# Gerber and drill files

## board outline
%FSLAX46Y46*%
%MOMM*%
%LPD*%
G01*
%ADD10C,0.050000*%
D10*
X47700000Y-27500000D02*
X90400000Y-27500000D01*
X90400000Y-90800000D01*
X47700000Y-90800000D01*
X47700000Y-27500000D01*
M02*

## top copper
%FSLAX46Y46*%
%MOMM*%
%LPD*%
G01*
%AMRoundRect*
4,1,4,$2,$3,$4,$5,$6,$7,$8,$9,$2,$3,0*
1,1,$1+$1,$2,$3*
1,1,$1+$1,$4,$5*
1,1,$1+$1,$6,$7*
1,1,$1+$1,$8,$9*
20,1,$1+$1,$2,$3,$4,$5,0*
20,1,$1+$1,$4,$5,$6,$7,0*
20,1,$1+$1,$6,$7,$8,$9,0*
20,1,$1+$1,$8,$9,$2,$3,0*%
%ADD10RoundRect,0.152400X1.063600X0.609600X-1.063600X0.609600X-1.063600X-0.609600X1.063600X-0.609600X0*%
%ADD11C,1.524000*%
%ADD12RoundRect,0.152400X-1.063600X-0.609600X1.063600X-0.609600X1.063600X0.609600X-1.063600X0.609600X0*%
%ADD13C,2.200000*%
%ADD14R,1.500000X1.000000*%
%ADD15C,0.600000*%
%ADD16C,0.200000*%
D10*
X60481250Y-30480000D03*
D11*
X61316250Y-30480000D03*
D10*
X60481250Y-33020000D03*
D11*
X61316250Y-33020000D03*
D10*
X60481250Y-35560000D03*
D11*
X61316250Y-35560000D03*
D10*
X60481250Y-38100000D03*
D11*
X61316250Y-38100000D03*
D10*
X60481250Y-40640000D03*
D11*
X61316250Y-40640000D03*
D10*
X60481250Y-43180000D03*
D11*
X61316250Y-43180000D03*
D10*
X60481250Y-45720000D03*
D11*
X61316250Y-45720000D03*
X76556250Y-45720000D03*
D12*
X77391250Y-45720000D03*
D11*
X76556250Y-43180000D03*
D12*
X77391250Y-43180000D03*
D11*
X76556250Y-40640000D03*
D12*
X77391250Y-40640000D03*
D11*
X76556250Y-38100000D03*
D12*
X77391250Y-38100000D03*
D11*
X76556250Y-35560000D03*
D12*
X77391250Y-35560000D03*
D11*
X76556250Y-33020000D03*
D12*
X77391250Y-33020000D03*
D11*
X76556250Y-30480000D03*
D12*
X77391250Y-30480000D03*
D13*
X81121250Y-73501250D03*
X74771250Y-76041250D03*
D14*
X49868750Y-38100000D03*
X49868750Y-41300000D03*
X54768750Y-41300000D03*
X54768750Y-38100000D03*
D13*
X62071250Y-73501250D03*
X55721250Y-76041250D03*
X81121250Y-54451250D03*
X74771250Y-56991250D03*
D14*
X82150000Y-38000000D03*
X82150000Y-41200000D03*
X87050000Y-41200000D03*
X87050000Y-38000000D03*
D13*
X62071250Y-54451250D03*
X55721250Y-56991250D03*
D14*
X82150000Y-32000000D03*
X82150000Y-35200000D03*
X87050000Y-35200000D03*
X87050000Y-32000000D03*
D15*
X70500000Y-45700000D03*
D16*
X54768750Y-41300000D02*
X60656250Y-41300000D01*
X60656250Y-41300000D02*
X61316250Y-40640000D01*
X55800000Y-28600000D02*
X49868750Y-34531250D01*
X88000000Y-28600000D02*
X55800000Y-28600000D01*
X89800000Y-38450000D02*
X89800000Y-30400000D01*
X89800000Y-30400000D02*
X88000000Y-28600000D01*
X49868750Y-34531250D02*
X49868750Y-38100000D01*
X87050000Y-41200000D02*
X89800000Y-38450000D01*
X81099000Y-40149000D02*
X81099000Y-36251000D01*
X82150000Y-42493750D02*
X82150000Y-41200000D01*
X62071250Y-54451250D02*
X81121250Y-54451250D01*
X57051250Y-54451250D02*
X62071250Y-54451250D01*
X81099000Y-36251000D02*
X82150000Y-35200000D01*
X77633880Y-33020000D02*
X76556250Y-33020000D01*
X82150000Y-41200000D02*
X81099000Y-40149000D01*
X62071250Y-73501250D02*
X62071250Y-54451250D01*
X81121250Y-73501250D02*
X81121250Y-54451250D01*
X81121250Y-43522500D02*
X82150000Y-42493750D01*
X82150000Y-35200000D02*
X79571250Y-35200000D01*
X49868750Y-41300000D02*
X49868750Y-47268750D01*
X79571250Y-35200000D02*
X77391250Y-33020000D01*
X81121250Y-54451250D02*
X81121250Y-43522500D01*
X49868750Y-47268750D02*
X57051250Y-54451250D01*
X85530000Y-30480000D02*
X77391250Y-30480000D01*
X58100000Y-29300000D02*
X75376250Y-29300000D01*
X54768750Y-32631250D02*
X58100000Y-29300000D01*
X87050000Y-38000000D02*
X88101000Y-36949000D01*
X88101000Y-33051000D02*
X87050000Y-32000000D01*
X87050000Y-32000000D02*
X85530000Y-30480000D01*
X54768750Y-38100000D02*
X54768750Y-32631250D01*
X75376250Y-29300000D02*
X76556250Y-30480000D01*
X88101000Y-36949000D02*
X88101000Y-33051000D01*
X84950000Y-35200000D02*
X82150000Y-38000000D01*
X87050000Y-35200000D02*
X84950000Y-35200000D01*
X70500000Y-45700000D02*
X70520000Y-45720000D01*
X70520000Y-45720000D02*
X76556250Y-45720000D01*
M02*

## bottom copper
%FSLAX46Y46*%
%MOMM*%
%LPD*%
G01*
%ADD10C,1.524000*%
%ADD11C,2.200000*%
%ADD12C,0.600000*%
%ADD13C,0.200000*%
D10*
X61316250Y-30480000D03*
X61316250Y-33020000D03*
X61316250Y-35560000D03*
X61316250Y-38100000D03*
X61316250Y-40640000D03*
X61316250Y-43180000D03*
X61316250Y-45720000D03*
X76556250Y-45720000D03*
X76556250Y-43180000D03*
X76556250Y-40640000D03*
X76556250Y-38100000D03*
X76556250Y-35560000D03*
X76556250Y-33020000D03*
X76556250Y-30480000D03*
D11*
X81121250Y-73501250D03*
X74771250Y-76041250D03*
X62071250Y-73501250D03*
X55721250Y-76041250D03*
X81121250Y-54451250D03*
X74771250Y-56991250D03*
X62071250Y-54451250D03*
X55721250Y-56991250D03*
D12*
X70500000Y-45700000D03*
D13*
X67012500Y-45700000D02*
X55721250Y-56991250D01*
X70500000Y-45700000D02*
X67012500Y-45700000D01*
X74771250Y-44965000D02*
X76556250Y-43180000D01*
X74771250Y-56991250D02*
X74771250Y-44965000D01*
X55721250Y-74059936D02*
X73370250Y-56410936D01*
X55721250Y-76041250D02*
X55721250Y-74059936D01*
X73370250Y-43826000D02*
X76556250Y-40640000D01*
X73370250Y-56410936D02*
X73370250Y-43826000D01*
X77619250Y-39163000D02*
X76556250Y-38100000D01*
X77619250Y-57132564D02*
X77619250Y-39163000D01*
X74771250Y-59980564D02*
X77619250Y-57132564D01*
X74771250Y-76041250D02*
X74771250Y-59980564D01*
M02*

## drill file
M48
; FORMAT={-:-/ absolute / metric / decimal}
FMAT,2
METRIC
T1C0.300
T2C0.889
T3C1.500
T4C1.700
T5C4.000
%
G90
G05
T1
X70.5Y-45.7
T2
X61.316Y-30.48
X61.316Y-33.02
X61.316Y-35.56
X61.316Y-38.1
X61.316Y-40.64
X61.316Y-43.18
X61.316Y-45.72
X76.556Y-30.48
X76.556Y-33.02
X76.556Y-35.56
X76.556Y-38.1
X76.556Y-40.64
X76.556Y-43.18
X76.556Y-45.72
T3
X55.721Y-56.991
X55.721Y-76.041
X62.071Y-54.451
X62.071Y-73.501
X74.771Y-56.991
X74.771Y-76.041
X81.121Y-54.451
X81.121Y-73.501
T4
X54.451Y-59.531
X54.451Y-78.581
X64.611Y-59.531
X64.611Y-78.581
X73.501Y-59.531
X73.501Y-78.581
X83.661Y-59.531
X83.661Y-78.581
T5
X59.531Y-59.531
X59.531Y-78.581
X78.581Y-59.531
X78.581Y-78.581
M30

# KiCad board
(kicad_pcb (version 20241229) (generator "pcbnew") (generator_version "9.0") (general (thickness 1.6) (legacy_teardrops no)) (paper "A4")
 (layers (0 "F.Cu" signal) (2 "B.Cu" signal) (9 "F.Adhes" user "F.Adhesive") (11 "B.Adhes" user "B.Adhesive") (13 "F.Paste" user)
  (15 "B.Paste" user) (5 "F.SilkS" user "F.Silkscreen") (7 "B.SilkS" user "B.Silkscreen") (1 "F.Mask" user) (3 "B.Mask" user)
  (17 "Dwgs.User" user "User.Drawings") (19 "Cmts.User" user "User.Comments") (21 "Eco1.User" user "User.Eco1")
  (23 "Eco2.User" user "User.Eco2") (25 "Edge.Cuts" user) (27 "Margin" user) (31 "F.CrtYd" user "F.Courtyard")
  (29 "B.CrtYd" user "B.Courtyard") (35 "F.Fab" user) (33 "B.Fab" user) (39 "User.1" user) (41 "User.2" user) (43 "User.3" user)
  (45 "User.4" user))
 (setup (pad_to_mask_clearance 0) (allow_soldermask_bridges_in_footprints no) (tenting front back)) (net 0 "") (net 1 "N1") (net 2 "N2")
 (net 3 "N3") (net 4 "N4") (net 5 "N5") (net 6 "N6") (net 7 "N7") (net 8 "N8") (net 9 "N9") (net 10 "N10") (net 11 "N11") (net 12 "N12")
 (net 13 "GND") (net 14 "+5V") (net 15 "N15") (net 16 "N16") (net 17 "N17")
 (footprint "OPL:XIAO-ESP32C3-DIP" (layer "F.Cu") (at 69.05625 38.1)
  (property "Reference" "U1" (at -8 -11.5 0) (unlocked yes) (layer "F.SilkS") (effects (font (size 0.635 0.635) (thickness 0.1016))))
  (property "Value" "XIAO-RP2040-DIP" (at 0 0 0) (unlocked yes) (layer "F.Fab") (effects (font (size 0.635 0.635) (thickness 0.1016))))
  (pad "1" smd roundrect (at -8.575 -7.62 180) (size 2.432 1.524) (layers "F.Cu" "F.Mask") (roundrect_rratio 0.1) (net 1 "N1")
   (thermal_bridge_angle 45))
  (pad "1" thru_hole circle (at -7.74 -7.62 180) (size 1.524 1.524) (drill 0.889) (layers "*.Cu" "*.Mask") (remove_unused_layers no)
   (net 1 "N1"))
  (pad "2" smd roundrect (at -8.575 -5.08 180) (size 2.432 1.524) (layers "F.Cu" "F.Mask") (roundrect_rratio 0.1) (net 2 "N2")
   (thermal_bridge_angle 45))
  (pad "2" thru_hole circle (at -7.74 -5.08 180) (size 1.524 1.524) (drill 0.889) (layers "*.Cu" "*.Mask") (remove_unused_layers no)
   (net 2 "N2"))
  (pad "3" smd roundrect (at -8.575 -2.54 180) (size 2.432 1.524) (layers "F.Cu" "F.Mask") (roundrect_rratio 0.1) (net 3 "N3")
   (thermal_bridge_angle 45))
  (pad "3" thru_hole circle (at -7.74 -2.54 180) (size 1.524 1.524) (drill 0.889) (layers "*.Cu" "*.Mask") (remove_unused_layers no)
   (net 3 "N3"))
  (pad "4" smd roundrect (at -8.575 0 180) (size 2.432 1.524) (layers "F.Cu" "F.Mask") (roundrect_rratio 0.1) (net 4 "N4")
   (thermal_bridge_angle 45))
  (pad "4" thru_hole circle (at -7.74 0 180) (size 1.524 1.524) (drill 0.889) (layers "*.Cu" "*.Mask") (remove_unused_layers no)
   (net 4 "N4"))
  (pad "5" smd roundrect (at -8.575 2.54 180) (size 2.432 1.524) (layers "F.Cu" "F.Mask") (roundrect_rratio 0.1) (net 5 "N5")
   (thermal_bridge_angle 45))
  (pad "5" thru_hole circle (at -7.74 2.54 180) (size 1.524 1.524) (drill 0.889) (layers "*.Cu" "*.Mask") (remove_unused_layers no)
   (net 5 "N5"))
  (pad "6" smd roundrect (at -8.575 5.08 180) (size 2.432 1.524) (layers "F.Cu" "F.Mask") (roundrect_rratio 0.1) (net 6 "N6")
   (thermal_bridge_angle 45))
  (pad "6" thru_hole circle (at -7.74 5.08 180) (size 1.524 1.524) (drill 0.889) (layers "*.Cu" "*.Mask") (remove_unused_layers no)
   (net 6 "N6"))
  (pad "7" smd roundrect (at -8.575 7.62 180) (size 2.432 1.524) (layers "F.Cu" "F.Mask") (roundrect_rratio 0.1) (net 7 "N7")
   (thermal_bridge_angle 45))
  (pad "7" thru_hole circle (at -7.74 7.62 180) (size 1.524 1.524) (drill 0.889) (layers "*.Cu" "*.Mask") (remove_unused_layers no)
   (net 7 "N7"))
  (pad "8" thru_hole circle (at 7.5 7.62) (size 1.524 1.524) (drill 0.889) (layers "*.Cu" "*.Mask") (remove_unused_layers no) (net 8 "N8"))
  (pad "8" smd roundrect (at 8.335 7.62) (size 2.432 1.524) (layers "F.Cu" "F.Mask") (roundrect_rratio 0.1) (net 8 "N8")
   (thermal_bridge_angle 45))
  (pad "9" thru_hole circle (at 7.5 5.08) (size 1.524 1.524) (drill 0.889) (layers "*.Cu" "*.Mask") (remove_unused_layers no) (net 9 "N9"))
  (pad "9" smd roundrect (at 8.335 5.08) (size 2.432 1.524) (layers "F.Cu" "F.Mask") (roundrect_rratio 0.1) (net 9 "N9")
   (thermal_bridge_angle 45))
  (pad "10" thru_hole circle (at 7.5 2.54) (size 1.524 1.524) (drill 0.889) (layers "*.Cu" "*.Mask") (remove_unused_layers no)
   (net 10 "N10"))
  (pad "10" smd roundrect (at 8.335 2.54) (size 2.432 1.524) (layers "F.Cu" "F.Mask") (roundrect_rratio 0.1) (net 10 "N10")
   (thermal_bridge_angle 45))
  (pad "11" thru_hole circle (at 7.5 0) (size 1.524 1.524) (drill 0.889) (layers "*.Cu" "*.Mask") (remove_unused_layers no) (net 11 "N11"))
  (pad "11" smd roundrect (at 8.335 0) (size 2.432 1.524) (layers "F.Cu" "F.Mask") (roundrect_rratio 0.1) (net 11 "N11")
   (thermal_bridge_angle 45))
  (pad "12" thru_hole circle (at 7.5 -2.54) (size 1.524 1.524) (drill 0.889) (layers "*.Cu" "*.Mask") (remove_unused_layers no)
   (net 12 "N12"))
  (pad "12" smd roundrect (at 8.335 -2.54) (size 2.432 1.524) (layers "F.Cu" "F.Mask") (roundrect_rratio 0.1) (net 12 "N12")
   (thermal_bridge_angle 45))
  (pad "13" thru_hole circle (at 7.5 -5.08) (size 1.524 1.524) (drill 0.889) (layers "*.Cu" "*.Mask") (remove_unused_layers no)
   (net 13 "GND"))
  (pad "13" smd roundrect (at 8.335 -5.08) (size 2.432 1.524) (layers "F.Cu" "F.Mask") (roundrect_rratio 0.1) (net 13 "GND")
   (thermal_bridge_angle 45))
  (pad "14" thru_hole circle (at 7.5 -7.62) (size 1.524 1.524) (drill 0.889) (layers "*.Cu" "*.Mask") (remove_unused_layers no)
   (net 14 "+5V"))
  (pad "14" smd roundrect (at 8.335 -7.62) (size 2.432 1.524) (layers "F.Cu" "F.Mask") (roundrect_rratio 0.1) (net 14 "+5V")
   (thermal_bridge_angle 45)))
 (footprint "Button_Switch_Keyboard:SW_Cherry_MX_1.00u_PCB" (layer "F.Cu") (at 81.12125 73.50125)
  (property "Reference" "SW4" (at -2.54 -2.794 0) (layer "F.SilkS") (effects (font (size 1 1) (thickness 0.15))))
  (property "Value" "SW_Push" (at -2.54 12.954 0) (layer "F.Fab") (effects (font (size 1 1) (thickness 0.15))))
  (pad "" np_thru_hole circle (at -7.62 5.08) (size 1.7 1.7) (drill 1.7) (layers "*.Cu" "*.Mask"))
  (pad "" np_thru_hole circle (at -2.54 5.08) (size 4 4) (drill 4) (layers "*.Cu" "*.Mask"))
  (pad "" np_thru_hole circle (at 2.54 5.08) (size 1.7 1.7) (drill 1.7) (layers "*.Cu" "*.Mask"))
  (pad "1" thru_hole circle (at 0 0) (size 2.2 2.2) (drill 1.5) (layers "*.Cu" "*.Mask") (remove_unused_layers no) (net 13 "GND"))
  (pad "2" thru_hole circle (at -6.35 2.54) (size 2.2 2.2) (drill 1.5) (layers "*.Cu" "*.Mask") (remove_unused_layers no) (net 11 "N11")))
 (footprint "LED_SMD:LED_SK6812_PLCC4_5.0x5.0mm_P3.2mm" (layer "F.Cu") (at 52.31875 39.7)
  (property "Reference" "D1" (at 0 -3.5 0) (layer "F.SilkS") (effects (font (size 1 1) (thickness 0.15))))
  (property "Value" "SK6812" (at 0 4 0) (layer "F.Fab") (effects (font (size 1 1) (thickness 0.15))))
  (pad "1" smd rect (at -2.45 -1.6 180) (size 1.5 1) (layers "F.Cu" "F.Mask" "F.Paste") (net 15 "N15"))
  (pad "2" smd rect (at -2.45 1.6 180) (size 1.5 1) (layers "F.Cu" "F.Mask" "F.Paste") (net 13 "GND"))
  (pad "3" smd rect (at 2.45 1.6 180) (size 1.5 1) (layers "F.Cu" "F.Mask" "F.Paste") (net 5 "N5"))
  (pad "4" smd rect (at 2.45 -1.6 180) (size 1.5 1) (layers "F.Cu" "F.Mask" "F.Paste") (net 14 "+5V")))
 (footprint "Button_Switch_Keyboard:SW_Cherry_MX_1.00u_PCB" (layer "F.Cu") (at 62.07125 73.50125)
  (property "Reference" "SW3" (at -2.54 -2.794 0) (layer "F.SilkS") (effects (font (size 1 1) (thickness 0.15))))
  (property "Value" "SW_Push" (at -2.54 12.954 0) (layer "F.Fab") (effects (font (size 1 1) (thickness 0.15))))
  (pad "" np_thru_hole circle (at -7.62 5.08) (size 1.7 1.7) (drill 1.7) (layers "*.Cu" "*.Mask"))
  (pad "" np_thru_hole circle (at -2.54 5.08) (size 4 4) (drill 4) (layers "*.Cu" "*.Mask"))
  (pad "" np_thru_hole circle (at 2.54 5.08) (size 1.7 1.7) (drill 1.7) (layers "*.Cu" "*.Mask"))
  (pad "1" thru_hole circle (at 0 0) (size 2.2 2.2) (drill 1.5) (layers "*.Cu" "*.Mask") (remove_unused_layers no) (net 13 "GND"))
  (pad "2" thru_hole circle (at -6.35 2.54) (size 2.2 2.2) (drill 1.5) (layers "*.Cu" "*.Mask") (remove_unused_layers no) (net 10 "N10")))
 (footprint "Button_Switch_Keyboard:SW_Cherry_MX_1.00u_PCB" (layer "F.Cu") (at 81.12125 54.45125)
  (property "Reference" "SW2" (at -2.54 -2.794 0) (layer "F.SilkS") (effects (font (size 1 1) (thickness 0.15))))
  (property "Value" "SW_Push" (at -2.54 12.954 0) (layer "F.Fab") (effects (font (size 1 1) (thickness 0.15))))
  (pad "" np_thru_hole circle (at -7.62 5.08) (size 1.7 1.7) (drill 1.7) (layers "*.Cu" "*.Mask"))
  (pad "" np_thru_hole circle (at -2.54 5.08) (size 4 4) (drill 4) (layers "*.Cu" "*.Mask"))
  (pad "" np_thru_hole circle (at 2.54 5.08) (size 1.7 1.7) (drill 1.7) (layers "*.Cu" "*.Mask"))
  (pad "1" thru_hole circle (at 0 0) (size 2.2 2.2) (drill 1.5) (layers "*.Cu" "*.Mask") (remove_unused_layers no) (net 13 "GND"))
  (pad "2" thru_hole circle (at -6.35 2.54) (size 2.2 2.2) (drill 1.5) (layers "*.Cu" "*.Mask") (remove_unused_layers no) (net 9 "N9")))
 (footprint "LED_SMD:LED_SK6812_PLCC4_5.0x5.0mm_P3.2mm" (layer "F.Cu") (at 84.6 39.6)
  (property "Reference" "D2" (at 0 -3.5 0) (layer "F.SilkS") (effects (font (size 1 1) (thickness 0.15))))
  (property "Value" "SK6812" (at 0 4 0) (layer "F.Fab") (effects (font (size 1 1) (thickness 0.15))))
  (pad "1" smd rect (at -2.45 -1.6 180) (size 1.5 1) (layers "F.Cu" "F.Mask" "F.Paste") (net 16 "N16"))
  (pad "2" smd rect (at -2.45 1.6 180) (size 1.5 1) (layers "F.Cu" "F.Mask" "F.Paste") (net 13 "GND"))
  (pad "3" smd rect (at 2.45 1.6 180) (size 1.5 1) (layers "F.Cu" "F.Mask" "F.Paste") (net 15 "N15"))
  (pad "4" smd rect (at 2.45 -1.6 180) (size 1.5 1) (layers "F.Cu" "F.Mask" "F.Paste") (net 14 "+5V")))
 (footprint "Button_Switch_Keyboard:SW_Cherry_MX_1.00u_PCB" (layer "F.Cu") (at 62.07125 54.45125)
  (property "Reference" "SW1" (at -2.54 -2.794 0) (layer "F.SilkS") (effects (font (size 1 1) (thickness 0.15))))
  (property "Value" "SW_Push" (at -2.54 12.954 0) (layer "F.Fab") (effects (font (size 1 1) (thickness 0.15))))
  (pad "" np_thru_hole circle (at -7.62 5.08) (size 1.7 1.7) (drill 1.7) (layers "*.Cu" "*.Mask"))
  (pad "" np_thru_hole circle (at -2.54 5.08) (size 4 4) (drill 4) (layers "*.Cu" "*.Mask"))
  (pad "" np_thru_hole circle (at 2.54 5.08) (size 1.7 1.7) (drill 1.7) (layers "*.Cu" "*.Mask"))
  (pad "1" thru_hole circle (at 0 0) (size 2.2 2.2) (drill 1.5) (layers "*.Cu" "*.Mask") (remove_unused_layers no) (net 13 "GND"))
  (pad "2" thru_hole circle (at -6.35 2.54) (size 2.2 2.2) (drill 1.5) (layers "*.Cu" "*.Mask") (remove_unused_layers no) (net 8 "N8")))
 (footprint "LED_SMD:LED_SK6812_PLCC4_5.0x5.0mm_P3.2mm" (layer "F.Cu") (at 84.6 33.6)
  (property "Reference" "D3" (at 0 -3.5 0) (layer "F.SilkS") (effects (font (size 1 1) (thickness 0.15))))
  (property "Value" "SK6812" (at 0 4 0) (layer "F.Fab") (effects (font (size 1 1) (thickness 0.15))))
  (pad "1" smd rect (at -2.45 -1.6 180) (size 1.5 1) (layers "F.Cu" "F.Mask" "F.Paste") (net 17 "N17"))
  (pad "2" smd rect (at -2.45 1.6 180) (size 1.5 1) (layers "F.Cu" "F.Mask" "F.Paste") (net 13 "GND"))
  (pad "3" smd rect (at 2.45 1.6 180) (size 1.5 1) (layers "F.Cu" "F.Mask" "F.Paste") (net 16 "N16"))
  (pad "4" smd rect (at 2.45 -1.6 180) (size 1.5 1) (layers "F.Cu" "F.Mask" "F.Paste") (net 14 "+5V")))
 (gr_rect (start 47.7 27.5) (end 90.4 90.8) (stroke (width 0.05) (type default)) (fill no) (layer "Edge.Cuts"))
 (segment (start 54.76875 41.3) (end 60.65625 41.3) (width 0.2) (layer "F.Cu") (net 5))
 (segment (start 60.65625 41.3) (end 61.31625 40.64) (width 0.2) (layer "F.Cu") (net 5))
 (segment (start 55.8 28.6) (end 49.86875 34.53125) (width 0.2) (layer "F.Cu") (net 15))
 (segment (start 88 28.6) (end 55.8 28.6) (width 0.2) (layer "F.Cu") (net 15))
 (segment (start 89.8 38.45) (end 89.8 30.4) (width 0.2) (layer "F.Cu") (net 15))
 (segment (start 89.8 30.4) (end 88 28.6) (width 0.2) (layer "F.Cu") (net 15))
 (segment (start 49.86875 34.53125) (end 49.86875 38.1) (width 0.2) (layer "F.Cu") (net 15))
 (segment (start 87.05 41.2) (end 89.8 38.45) (width 0.2) (layer "F.Cu") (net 15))
 (segment (start 81.099 40.149) (end 81.099 36.251) (width 0.2) (layer "F.Cu") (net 13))
 (segment (start 82.15 42.49375) (end 82.15 41.2) (width 0.2) (layer "F.Cu") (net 13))
 (segment (start 62.07125 54.45125) (end 81.12125 54.45125) (width 0.2) (layer "F.Cu") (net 13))
 (segment (start 57.05125 54.45125) (end 62.07125 54.45125) (width 0.2) (layer "F.Cu") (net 13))
 (segment (start 81.099 36.251) (end 82.15 35.2) (width 0.2) (layer "F.Cu") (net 13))
 (segment (start 77.63388 33.02) (end 76.55625 33.02) (width 0.2) (layer "F.Cu") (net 13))
 (segment (start 82.15 41.2) (end 81.099 40.149) (width 0.2) (layer "F.Cu") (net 13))
 (segment (start 62.07125 73.50125) (end 62.07125 54.45125) (width 0.2) (layer "F.Cu") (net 13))
 (segment (start 81.12125 73.50125) (end 81.12125 54.45125) (width 0.2) (layer "F.Cu") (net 13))
 (segment (start 81.12125 43.5225) (end 82.15 42.49375) (width 0.2) (layer "F.Cu") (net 13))
 (segment (start 82.15 35.2) (end 79.57125 35.2) (width 0.2) (layer "F.Cu") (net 13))
 (segment (start 49.86875 41.3) (end 49.86875 47.26875) (width 0.2) (layer "F.Cu") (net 13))
 (segment (start 79.57125 35.2) (end 77.39125 33.02) (width 0.2) (layer "F.Cu") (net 13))
 (segment (start 81.12125 54.45125) (end 81.12125 43.5225) (width 0.2) (layer "F.Cu") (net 13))
 (segment (start 49.86875 47.26875) (end 57.05125 54.45125) (width 0.2) (layer "F.Cu") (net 13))
 (segment (start 85.53 30.48) (end 77.39125 30.48) (width 0.2) (layer "F.Cu") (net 14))
 (segment (start 58.1 29.3) (end 75.37625 29.3) (width 0.2) (layer "F.Cu") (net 14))
 (segment (start 54.76875 32.63125) (end 58.1 29.3) (width 0.2) (layer "F.Cu") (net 14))
 (segment (start 87.05 38) (end 88.101 36.949) (width 0.2) (layer "F.Cu") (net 14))
 (segment (start 88.101 33.051) (end 87.05 32) (width 0.2) (layer "F.Cu") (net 14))
 (segment (start 87.05 32) (end 85.53 30.48) (width 0.2) (layer "F.Cu") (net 14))
 (segment (start 54.76875 38.1) (end 54.76875 32.63125) (width 0.2) (layer "F.Cu") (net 14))
 (segment (start 75.37625 29.3) (end 76.55625 30.48) (width 0.2) (layer "F.Cu") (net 14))
 (segment (start 88.101 36.949) (end 88.101 33.051) (width 0.2) (layer "F.Cu") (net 14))
 (segment (start 84.95 35.2) (end 82.15 38) (width 0.2) (layer "F.Cu") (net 16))
 (segment (start 87.05 35.2) (end 84.95 35.2) (width 0.2) (layer "F.Cu") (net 16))
 (segment (start 70.5 45.7) (end 70.52 45.72) (width 0.2) (layer "F.Cu") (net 8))
 (segment (start 70.52 45.72) (end 76.55625 45.72) (width 0.2) (layer "F.Cu") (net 8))
 (via (at 70.5 45.7) (size 0.6) (drill 0.3) (layers "F.Cu" "B.Cu") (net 8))
 (segment (start 67.0125 45.7) (end 55.72125 56.99125) (width 0.2) (layer "B.Cu") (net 8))
 (segment (start 70.5 45.7) (end 67.0125 45.7) (width 0.2) (layer "B.Cu") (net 8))
 (segment (start 74.77125 44.965) (end 76.55625 43.18) (width 0.2) (layer "B.Cu") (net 9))
 (segment (start 74.77125 56.99125) (end 74.77125 44.965) (width 0.2) (layer "B.Cu") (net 9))
 (segment (start 55.72125 74.059936) (end 73.37025 56.410936) (width 0.2) (layer "B.Cu") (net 10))
 (segment (start 55.72125 76.04125) (end 55.72125 74.059936) (width 0.2) (layer "B.Cu") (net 10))
 (segment (start 73.37025 43.826) (end 76.55625 40.64) (width 0.2) (layer "B.Cu") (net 10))
 (segment (start 73.37025 56.410936) (end 73.37025 43.826) (width 0.2) (layer "B.Cu") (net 10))
 (segment (start 77.61925 39.163) (end 76.55625 38.1) (width 0.2) (layer "B.Cu") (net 11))
 (segment (start 77.61925 57.132564) (end 77.61925 39.163) (width 0.2) (layer "B.Cu") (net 11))
 (segment (start 74.77125 59.980564) (end 77.61925 57.132564) (width 0.2) (layer "B.Cu") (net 11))
 (segment (start 74.77125 76.04125) (end 74.77125 59.980564) (width 0.2) (layer "B.Cu") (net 11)))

